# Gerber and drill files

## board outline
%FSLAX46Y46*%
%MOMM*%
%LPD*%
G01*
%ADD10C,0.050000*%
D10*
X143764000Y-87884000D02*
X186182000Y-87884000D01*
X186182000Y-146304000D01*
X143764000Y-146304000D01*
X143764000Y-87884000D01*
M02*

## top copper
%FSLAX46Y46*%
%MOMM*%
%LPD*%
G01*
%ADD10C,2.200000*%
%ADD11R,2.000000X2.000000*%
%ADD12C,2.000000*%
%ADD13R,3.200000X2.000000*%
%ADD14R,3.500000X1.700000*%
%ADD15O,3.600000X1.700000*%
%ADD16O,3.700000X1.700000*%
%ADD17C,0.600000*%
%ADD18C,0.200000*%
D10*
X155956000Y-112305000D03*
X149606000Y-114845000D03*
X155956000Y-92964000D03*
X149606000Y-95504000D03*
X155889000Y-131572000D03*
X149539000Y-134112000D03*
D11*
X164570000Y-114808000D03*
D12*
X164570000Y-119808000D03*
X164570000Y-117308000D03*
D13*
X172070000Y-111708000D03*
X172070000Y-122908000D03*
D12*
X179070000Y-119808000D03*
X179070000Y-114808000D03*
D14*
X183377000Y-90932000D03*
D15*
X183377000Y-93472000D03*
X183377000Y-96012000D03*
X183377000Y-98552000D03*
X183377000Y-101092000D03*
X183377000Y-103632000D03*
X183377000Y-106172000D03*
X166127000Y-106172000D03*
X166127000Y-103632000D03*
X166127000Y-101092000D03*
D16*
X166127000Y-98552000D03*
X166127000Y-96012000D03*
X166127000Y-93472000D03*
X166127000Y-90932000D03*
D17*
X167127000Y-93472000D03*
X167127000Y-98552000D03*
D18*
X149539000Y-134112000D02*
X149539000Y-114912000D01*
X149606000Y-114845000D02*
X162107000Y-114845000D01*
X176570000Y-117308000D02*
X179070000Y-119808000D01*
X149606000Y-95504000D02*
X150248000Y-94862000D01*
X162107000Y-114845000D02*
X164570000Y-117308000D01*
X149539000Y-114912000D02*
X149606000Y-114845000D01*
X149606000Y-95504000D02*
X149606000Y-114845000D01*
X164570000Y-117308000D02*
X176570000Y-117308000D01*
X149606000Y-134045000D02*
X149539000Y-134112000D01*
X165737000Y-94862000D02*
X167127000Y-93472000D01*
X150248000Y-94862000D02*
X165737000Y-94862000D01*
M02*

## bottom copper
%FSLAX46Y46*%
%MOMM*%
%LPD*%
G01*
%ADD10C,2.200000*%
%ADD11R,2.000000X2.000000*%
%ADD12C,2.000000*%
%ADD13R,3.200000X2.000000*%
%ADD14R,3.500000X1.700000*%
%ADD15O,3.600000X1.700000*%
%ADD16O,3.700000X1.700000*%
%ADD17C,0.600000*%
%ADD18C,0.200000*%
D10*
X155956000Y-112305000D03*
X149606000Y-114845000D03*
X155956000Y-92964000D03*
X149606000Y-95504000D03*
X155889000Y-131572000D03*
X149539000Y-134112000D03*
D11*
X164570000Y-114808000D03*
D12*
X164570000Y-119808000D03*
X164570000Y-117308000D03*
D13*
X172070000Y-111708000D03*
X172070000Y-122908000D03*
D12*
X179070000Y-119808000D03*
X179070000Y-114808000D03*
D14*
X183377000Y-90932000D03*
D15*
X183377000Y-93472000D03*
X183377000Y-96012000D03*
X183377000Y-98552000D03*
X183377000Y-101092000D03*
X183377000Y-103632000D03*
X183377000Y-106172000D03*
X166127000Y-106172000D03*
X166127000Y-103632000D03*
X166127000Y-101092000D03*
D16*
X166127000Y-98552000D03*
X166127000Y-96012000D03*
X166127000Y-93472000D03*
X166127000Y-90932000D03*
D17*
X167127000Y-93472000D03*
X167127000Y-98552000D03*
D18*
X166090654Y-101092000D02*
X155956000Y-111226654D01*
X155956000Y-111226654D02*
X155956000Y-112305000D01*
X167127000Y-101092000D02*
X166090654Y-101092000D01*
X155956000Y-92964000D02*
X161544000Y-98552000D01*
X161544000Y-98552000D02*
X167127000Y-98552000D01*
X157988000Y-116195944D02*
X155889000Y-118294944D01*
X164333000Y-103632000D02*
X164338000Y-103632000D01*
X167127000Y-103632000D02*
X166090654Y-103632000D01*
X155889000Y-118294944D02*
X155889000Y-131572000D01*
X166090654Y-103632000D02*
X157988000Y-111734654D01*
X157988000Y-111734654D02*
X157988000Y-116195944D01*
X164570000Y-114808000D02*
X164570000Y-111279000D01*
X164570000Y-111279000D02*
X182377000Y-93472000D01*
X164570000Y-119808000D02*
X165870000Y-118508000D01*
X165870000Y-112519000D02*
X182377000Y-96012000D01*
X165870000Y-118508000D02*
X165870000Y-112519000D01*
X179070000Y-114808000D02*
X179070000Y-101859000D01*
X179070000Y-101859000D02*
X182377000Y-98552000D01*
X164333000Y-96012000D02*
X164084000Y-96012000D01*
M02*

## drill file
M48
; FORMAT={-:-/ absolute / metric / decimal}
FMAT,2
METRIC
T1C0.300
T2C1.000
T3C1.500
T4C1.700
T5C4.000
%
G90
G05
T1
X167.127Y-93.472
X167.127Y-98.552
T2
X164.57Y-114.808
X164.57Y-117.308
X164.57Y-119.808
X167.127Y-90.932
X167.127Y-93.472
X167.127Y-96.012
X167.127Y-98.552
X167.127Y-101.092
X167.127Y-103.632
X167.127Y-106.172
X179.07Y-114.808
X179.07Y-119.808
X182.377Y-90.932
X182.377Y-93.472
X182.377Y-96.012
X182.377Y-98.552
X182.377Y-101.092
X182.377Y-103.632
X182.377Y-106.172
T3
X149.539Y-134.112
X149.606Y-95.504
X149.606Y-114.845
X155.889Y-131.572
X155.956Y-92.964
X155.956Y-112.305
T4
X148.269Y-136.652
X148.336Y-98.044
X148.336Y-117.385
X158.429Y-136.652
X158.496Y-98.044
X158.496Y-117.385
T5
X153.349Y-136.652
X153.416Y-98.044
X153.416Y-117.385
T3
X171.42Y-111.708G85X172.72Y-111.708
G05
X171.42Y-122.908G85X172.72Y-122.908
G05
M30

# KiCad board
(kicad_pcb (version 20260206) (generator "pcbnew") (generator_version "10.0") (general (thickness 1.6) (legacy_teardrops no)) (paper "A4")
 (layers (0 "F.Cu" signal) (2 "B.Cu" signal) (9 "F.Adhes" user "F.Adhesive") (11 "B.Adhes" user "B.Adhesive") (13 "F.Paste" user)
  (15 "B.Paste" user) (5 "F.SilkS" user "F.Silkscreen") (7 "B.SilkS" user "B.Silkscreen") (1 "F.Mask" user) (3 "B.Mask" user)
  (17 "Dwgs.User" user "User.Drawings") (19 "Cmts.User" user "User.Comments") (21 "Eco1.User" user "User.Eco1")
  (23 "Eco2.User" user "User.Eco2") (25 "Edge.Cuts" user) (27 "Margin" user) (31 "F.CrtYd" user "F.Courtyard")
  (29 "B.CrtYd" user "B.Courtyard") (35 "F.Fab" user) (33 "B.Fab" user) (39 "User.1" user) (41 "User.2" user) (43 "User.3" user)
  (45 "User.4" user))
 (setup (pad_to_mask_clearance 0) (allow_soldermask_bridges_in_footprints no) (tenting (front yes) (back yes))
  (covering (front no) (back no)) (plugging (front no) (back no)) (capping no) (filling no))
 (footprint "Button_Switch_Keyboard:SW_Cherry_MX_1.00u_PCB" (layer "F.Cu") (at 155.956 112.305)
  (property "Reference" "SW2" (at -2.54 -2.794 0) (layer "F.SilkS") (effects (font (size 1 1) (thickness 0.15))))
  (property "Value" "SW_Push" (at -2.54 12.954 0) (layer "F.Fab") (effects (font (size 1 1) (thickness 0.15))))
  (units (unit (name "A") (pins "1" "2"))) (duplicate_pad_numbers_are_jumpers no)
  (pad "" np_thru_hole circle (at -7.62 5.08) (size 1.7 1.7) (drill 1.7) (layers "*.Cu" "*.Mask"))
  (pad "" np_thru_hole circle (at -2.54 5.08) (size 4 4) (drill 4) (layers "*.Cu" "*.Mask"))
  (pad "" np_thru_hole circle (at 2.54 5.08) (size 1.7 1.7) (drill 1.7) (layers "*.Cu" "*.Mask"))
  (pad "1" thru_hole circle (at 0 0) (size 2.2 2.2) (drill 1.5) (layers "*.Cu" "*.Mask") (remove_unused_layers no)
   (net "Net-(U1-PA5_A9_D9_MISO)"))
  (pad "2" thru_hole circle (at -6.35 2.54) (size 2.2 2.2) (drill 1.5) (layers "*.Cu" "*.Mask") (remove_unused_layers no) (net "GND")))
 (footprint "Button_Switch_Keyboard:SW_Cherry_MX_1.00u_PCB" (layer "F.Cu") (at 155.956 92.964)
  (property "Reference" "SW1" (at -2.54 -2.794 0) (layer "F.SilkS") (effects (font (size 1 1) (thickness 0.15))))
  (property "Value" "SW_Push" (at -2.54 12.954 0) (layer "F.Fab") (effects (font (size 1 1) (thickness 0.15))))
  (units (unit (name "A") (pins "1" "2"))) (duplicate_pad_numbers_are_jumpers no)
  (pad "" np_thru_hole circle (at -7.62 5.08) (size 1.7 1.7) (drill 1.7) (layers "*.Cu" "*.Mask"))
  (pad "" np_thru_hole circle (at -2.54 5.08) (size 4 4) (drill 4) (layers "*.Cu" "*.Mask"))
  (pad "" np_thru_hole circle (at 2.54 5.08) (size 1.7 1.7) (drill 1.7) (layers "*.Cu" "*.Mask"))
  (pad "1" thru_hole circle (at 0 0) (size 2.2 2.2) (drill 1.5) (layers "*.Cu" "*.Mask") (remove_unused_layers no)
   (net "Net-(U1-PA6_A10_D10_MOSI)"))
  (pad "2" thru_hole circle (at -6.35 2.54) (size 2.2 2.2) (drill 1.5) (layers "*.Cu" "*.Mask") (remove_unused_layers no) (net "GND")))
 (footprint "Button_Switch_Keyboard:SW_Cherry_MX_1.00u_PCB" (layer "F.Cu") (at 155.889 131.572)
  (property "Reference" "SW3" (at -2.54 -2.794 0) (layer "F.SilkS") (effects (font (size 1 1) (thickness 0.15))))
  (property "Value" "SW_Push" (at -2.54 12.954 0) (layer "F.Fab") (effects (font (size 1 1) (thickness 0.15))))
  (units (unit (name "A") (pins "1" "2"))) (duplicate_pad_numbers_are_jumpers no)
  (pad "" np_thru_hole circle (at -7.62 5.08) (size 1.7 1.7) (drill 1.7) (layers "*.Cu" "*.Mask"))
  (pad "" np_thru_hole circle (at -2.54 5.08) (size 4 4) (drill 4) (layers "*.Cu" "*.Mask"))
  (pad "" np_thru_hole circle (at 2.54 5.08) (size 1.7 1.7) (drill 1.7) (layers "*.Cu" "*.Mask"))
  (pad "1" thru_hole circle (at 0 0) (size 2.2 2.2) (drill 1.5) (layers "*.Cu" "*.Mask") (remove_unused_layers no)
   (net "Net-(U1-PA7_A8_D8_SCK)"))
  (pad "2" thru_hole circle (at -6.35 2.54) (size 2.2 2.2) (drill 1.5) (layers "*.Cu" "*.Mask") (remove_unused_layers no) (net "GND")))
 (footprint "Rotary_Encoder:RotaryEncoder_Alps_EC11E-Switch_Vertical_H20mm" (layer "F.Cu") (at 164.57 114.808)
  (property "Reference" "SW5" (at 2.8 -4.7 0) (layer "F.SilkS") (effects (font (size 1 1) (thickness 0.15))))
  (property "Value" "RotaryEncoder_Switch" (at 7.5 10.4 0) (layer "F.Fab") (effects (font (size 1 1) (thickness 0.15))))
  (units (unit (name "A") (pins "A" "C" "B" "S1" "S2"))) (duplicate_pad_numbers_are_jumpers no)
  (pad "A" thru_hole rect (at 0 0) (size 2 2) (drill 1) (layers "*.Cu" "*.Mask") (remove_unused_layers no) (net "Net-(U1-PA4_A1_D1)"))
  (pad "B" thru_hole circle (at 0 5) (size 2 2) (drill 1) (layers "*.Cu" "*.Mask") (remove_unused_layers no) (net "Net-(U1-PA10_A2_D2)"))
  (pad "C" thru_hole circle (at 0 2.5) (size 2 2) (drill 1) (layers "*.Cu" "*.Mask") (remove_unused_layers no) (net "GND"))
  (pad "MP" thru_hole rect (at 7.5 -3.1) (size 3.2 2) (drill oval 2.8 1.5) (layers "*.Cu" "*.Mask") (remove_unused_layers no))
  (pad "MP" thru_hole rect (at 7.5 8.1) (size 3.2 2) (drill oval 2.8 1.5) (layers "*.Cu" "*.Mask") (remove_unused_layers no))
  (pad "S1" thru_hole circle (at 14.5 5) (size 2 2) (drill 1) (layers "*.Cu" "*.Mask") (remove_unused_layers no) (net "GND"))
  (pad "S2" thru_hole circle (at 14.5 0) (size 2 2) (drill 1) (layers "*.Cu" "*.Mask") (remove_unused_layers no) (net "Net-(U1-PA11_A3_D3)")))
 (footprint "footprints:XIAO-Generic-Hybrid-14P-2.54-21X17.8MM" (layer "B.Cu") (at 174.752 98.552 180)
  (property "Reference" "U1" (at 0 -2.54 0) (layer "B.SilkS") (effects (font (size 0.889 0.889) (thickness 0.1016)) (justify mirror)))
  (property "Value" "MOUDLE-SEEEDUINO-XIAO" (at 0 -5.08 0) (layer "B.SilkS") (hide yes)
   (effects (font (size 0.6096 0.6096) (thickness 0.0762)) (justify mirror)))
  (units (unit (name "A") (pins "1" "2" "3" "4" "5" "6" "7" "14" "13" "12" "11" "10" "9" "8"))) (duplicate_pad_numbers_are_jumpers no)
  (pad "1" thru_hole rect (at -7.625 7.62 180) (size 3.5 1.7) (drill 1 (offset -1 0)) (layers "*.Cu" "*.Mask") (remove_unused_layers no)
   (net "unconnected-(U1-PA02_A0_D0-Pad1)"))
  (pad "2" thru_hole oval (at -7.625 5.08 180) (size 3.6 1.7) (drill 1 (offset -1 0)) (layers "*.Cu" "*.Mask") (remove_unused_layers no)
   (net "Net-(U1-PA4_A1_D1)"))
  (pad "3" thru_hole oval (at -7.625 2.54 180) (size 3.6 1.7) (drill 1 (offset -1 0)) (layers "*.Cu" "*.Mask") (remove_unused_layers no)
   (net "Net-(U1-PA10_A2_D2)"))
  (pad "4" thru_hole oval (at -7.625 0 180) (size 3.6 1.7) (drill 1 (offset -1 0)) (layers "*.Cu" "*.Mask") (remove_unused_layers no)
   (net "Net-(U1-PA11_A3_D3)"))
  (pad "5" thru_hole oval (at -7.625 -2.54 180) (size 3.6 1.7) (drill 1 (offset -1 0)) (layers "*.Cu" "*.Mask") (remove_unused_layers no)
   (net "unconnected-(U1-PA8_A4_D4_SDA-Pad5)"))
  (pad "6" thru_hole oval (at -7.625 -5.08) (size 3.6 1.7) (drill 1 (offset 1 0)) (layers "*.Cu" "*.Mask") (remove_unused_layers no)
   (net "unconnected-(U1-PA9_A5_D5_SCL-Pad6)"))
  (pad "7" thru_hole oval (at -7.625 -7.62 180) (size 3.6 1.7) (drill 1 (offset -1 0)) (layers "*.Cu" "*.Mask") (remove_unused_layers no)
   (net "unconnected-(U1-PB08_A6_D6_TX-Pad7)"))
  (pad "8" thru_hole oval (at 7.625 -7.62 180) (size 3.6 1.7) (drill 1 (offset 1 0)) (layers "*.Cu" "*.Mask") (remove_unused_layers no)
   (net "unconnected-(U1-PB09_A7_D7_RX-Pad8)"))
  (pad "9" thru_hole oval (at 7.625 -5.08 180) (size 3.6 1.7) (drill 1 (offset 1 0)) (layers "*.Cu" "*.Mask") (remove_unused_layers no)
   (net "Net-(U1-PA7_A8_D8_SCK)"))
  (pad "10" thru_hole oval (at 7.625 -2.54 180) (size 3.6 1.7) (drill 1 (offset 1 0)) (layers "*.Cu" "*.Mask") (remove_unused_layers no)
   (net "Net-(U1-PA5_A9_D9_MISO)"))
  (pad "11" thru_hole oval (at 7.625 0 180) (size 3.7 1.7) (drill 1 (offset 1 0)) (layers "*.Cu" "*.Mask") (remove_unused_layers no)
   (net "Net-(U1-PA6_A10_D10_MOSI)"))
  (pad "12" thru_hole oval (at 7.625 2.54 180) (size 3.7 1.7) (drill 1 (offset 1 0)) (layers "*.Cu" "*.Mask") (remove_unused_layers no)
   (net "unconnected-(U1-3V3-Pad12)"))
  (pad "13" thru_hole oval (at 7.625 5.08 180) (size 3.7 1.7) (drill 1 (offset 1 0)) (layers "*.Cu" "*.Mask") (remove_unused_layers no)
   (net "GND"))
  (pad "14" thru_hole oval (at 7.625 7.62 180) (size 3.7 1.7) (drill 1 (offset 1 0)) (layers "*.Cu" "*.Mask") (remove_unused_layers no)
   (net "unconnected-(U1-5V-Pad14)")))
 (gr_rect (start 143.764 87.884) (end 186.182 146.304) (stroke (width 0.05) (type default)) (fill no) (layer "Edge.Cuts"))
 (segment (start 166.090654 101.092) (end 155.956 111.226654) (width 0.2) (layer "B.Cu") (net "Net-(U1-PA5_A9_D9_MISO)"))
 (segment (start 155.956 111.226654) (end 155.956 112.305) (width 0.2) (layer "B.Cu") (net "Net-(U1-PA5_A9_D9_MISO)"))
 (segment (start 167.127 101.092) (end 166.090654 101.092) (width 0.2) (layer "B.Cu") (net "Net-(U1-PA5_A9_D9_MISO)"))
 (segment (start 149.539 134.112) (end 149.539 114.912) (width 0.2) (layer "F.Cu") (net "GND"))
 (segment (start 149.606 114.845) (end 162.107 114.845) (width 0.2) (layer "F.Cu") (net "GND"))
 (segment (start 176.57 117.308) (end 179.07 119.808) (width 0.2) (layer "F.Cu") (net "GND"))
 (segment (start 149.606 95.504) (end 150.248 94.862) (width 0.2) (layer "F.Cu") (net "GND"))
 (segment (start 162.107 114.845) (end 164.57 117.308) (width 0.2) (layer "F.Cu") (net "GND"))
 (segment (start 149.539 114.912) (end 149.606 114.845) (width 0.2) (layer "F.Cu") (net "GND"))
 (segment (start 149.606 95.504) (end 149.606 114.845) (width 0.2) (layer "F.Cu") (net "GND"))
 (segment (start 164.57 117.308) (end 176.57 117.308) (width 0.2) (layer "F.Cu") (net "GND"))
 (segment (start 149.606 134.045) (end 149.539 134.112) (width 0.2) (layer "F.Cu") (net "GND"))
 (segment (start 165.737 94.862) (end 167.127 93.472) (width 0.2) (layer "F.Cu") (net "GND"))
 (segment (start 150.248 94.862) (end 165.737 94.862) (width 0.2) (layer "F.Cu") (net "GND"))
 (via (at 167.127 93.472) (size 0.6) (drill 0.3) (layers "F.Cu" "B.Cu") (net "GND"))
 (via (at 167.127 98.552) (size 0.6) (drill 0.3) (layers "F.Cu" "B.Cu") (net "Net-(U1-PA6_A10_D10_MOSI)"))
 (segment (start 155.956 92.964) (end 161.544 98.552) (width 0.2) (layer "B.Cu") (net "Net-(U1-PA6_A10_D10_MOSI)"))
 (segment (start 161.544 98.552) (end 167.127 98.552) (width 0.2) (layer "B.Cu") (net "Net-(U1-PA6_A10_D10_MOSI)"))
 (segment (start 157.988 116.195944) (end 155.889 118.294944) (width 0.2) (layer "B.Cu") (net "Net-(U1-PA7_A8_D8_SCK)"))
 (segment (start 164.333 103.632) (end 164.338 103.632) (width 0.2) (layer "B.Cu") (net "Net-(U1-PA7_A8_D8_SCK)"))
 (segment (start 167.127 103.632) (end 166.090654 103.632) (width 0.2) (layer "B.Cu") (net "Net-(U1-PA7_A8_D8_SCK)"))
 (segment (start 155.889 118.294944) (end 155.889 131.572) (width 0.2) (layer "B.Cu") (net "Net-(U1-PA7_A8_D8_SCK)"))
 (segment (start 166.090654 103.632) (end 157.988 111.734654) (width 0.2) (layer "B.Cu") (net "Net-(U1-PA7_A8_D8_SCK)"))
 (segment (start 157.988 111.734654) (end 157.988 116.195944) (width 0.2) (layer "B.Cu") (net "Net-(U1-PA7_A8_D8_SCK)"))
 (segment (start 164.57 114.808) (end 164.57 111.279) (width 0.2) (layer "B.Cu") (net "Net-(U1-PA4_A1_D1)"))
 (segment (start 164.57 111.279) (end 182.377 93.472) (width 0.2) (layer "B.Cu") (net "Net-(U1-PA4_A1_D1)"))
 (segment (start 164.57 119.808) (end 165.87 118.508) (width 0.2) (layer "B.Cu") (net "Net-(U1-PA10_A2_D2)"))
 (segment (start 165.87 112.519) (end 182.377 96.012) (width 0.2) (layer "B.Cu") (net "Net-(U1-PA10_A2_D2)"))
 (segment (start 165.87 118.508) (end 165.87 112.519) (width 0.2) (layer "B.Cu") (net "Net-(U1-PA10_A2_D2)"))
 (segment (start 179.07 114.808) (end 179.07 101.859) (width 0.2) (layer "B.Cu") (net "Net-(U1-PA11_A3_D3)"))
 (segment (start 179.07 101.859) (end 182.377 98.552) (width 0.2) (layer "B.Cu") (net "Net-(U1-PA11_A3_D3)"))
 (segment (start 164.333 96.012) (end 164.084 96.012) (width 0.2) (layer "B.Cu") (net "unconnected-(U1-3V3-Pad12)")))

